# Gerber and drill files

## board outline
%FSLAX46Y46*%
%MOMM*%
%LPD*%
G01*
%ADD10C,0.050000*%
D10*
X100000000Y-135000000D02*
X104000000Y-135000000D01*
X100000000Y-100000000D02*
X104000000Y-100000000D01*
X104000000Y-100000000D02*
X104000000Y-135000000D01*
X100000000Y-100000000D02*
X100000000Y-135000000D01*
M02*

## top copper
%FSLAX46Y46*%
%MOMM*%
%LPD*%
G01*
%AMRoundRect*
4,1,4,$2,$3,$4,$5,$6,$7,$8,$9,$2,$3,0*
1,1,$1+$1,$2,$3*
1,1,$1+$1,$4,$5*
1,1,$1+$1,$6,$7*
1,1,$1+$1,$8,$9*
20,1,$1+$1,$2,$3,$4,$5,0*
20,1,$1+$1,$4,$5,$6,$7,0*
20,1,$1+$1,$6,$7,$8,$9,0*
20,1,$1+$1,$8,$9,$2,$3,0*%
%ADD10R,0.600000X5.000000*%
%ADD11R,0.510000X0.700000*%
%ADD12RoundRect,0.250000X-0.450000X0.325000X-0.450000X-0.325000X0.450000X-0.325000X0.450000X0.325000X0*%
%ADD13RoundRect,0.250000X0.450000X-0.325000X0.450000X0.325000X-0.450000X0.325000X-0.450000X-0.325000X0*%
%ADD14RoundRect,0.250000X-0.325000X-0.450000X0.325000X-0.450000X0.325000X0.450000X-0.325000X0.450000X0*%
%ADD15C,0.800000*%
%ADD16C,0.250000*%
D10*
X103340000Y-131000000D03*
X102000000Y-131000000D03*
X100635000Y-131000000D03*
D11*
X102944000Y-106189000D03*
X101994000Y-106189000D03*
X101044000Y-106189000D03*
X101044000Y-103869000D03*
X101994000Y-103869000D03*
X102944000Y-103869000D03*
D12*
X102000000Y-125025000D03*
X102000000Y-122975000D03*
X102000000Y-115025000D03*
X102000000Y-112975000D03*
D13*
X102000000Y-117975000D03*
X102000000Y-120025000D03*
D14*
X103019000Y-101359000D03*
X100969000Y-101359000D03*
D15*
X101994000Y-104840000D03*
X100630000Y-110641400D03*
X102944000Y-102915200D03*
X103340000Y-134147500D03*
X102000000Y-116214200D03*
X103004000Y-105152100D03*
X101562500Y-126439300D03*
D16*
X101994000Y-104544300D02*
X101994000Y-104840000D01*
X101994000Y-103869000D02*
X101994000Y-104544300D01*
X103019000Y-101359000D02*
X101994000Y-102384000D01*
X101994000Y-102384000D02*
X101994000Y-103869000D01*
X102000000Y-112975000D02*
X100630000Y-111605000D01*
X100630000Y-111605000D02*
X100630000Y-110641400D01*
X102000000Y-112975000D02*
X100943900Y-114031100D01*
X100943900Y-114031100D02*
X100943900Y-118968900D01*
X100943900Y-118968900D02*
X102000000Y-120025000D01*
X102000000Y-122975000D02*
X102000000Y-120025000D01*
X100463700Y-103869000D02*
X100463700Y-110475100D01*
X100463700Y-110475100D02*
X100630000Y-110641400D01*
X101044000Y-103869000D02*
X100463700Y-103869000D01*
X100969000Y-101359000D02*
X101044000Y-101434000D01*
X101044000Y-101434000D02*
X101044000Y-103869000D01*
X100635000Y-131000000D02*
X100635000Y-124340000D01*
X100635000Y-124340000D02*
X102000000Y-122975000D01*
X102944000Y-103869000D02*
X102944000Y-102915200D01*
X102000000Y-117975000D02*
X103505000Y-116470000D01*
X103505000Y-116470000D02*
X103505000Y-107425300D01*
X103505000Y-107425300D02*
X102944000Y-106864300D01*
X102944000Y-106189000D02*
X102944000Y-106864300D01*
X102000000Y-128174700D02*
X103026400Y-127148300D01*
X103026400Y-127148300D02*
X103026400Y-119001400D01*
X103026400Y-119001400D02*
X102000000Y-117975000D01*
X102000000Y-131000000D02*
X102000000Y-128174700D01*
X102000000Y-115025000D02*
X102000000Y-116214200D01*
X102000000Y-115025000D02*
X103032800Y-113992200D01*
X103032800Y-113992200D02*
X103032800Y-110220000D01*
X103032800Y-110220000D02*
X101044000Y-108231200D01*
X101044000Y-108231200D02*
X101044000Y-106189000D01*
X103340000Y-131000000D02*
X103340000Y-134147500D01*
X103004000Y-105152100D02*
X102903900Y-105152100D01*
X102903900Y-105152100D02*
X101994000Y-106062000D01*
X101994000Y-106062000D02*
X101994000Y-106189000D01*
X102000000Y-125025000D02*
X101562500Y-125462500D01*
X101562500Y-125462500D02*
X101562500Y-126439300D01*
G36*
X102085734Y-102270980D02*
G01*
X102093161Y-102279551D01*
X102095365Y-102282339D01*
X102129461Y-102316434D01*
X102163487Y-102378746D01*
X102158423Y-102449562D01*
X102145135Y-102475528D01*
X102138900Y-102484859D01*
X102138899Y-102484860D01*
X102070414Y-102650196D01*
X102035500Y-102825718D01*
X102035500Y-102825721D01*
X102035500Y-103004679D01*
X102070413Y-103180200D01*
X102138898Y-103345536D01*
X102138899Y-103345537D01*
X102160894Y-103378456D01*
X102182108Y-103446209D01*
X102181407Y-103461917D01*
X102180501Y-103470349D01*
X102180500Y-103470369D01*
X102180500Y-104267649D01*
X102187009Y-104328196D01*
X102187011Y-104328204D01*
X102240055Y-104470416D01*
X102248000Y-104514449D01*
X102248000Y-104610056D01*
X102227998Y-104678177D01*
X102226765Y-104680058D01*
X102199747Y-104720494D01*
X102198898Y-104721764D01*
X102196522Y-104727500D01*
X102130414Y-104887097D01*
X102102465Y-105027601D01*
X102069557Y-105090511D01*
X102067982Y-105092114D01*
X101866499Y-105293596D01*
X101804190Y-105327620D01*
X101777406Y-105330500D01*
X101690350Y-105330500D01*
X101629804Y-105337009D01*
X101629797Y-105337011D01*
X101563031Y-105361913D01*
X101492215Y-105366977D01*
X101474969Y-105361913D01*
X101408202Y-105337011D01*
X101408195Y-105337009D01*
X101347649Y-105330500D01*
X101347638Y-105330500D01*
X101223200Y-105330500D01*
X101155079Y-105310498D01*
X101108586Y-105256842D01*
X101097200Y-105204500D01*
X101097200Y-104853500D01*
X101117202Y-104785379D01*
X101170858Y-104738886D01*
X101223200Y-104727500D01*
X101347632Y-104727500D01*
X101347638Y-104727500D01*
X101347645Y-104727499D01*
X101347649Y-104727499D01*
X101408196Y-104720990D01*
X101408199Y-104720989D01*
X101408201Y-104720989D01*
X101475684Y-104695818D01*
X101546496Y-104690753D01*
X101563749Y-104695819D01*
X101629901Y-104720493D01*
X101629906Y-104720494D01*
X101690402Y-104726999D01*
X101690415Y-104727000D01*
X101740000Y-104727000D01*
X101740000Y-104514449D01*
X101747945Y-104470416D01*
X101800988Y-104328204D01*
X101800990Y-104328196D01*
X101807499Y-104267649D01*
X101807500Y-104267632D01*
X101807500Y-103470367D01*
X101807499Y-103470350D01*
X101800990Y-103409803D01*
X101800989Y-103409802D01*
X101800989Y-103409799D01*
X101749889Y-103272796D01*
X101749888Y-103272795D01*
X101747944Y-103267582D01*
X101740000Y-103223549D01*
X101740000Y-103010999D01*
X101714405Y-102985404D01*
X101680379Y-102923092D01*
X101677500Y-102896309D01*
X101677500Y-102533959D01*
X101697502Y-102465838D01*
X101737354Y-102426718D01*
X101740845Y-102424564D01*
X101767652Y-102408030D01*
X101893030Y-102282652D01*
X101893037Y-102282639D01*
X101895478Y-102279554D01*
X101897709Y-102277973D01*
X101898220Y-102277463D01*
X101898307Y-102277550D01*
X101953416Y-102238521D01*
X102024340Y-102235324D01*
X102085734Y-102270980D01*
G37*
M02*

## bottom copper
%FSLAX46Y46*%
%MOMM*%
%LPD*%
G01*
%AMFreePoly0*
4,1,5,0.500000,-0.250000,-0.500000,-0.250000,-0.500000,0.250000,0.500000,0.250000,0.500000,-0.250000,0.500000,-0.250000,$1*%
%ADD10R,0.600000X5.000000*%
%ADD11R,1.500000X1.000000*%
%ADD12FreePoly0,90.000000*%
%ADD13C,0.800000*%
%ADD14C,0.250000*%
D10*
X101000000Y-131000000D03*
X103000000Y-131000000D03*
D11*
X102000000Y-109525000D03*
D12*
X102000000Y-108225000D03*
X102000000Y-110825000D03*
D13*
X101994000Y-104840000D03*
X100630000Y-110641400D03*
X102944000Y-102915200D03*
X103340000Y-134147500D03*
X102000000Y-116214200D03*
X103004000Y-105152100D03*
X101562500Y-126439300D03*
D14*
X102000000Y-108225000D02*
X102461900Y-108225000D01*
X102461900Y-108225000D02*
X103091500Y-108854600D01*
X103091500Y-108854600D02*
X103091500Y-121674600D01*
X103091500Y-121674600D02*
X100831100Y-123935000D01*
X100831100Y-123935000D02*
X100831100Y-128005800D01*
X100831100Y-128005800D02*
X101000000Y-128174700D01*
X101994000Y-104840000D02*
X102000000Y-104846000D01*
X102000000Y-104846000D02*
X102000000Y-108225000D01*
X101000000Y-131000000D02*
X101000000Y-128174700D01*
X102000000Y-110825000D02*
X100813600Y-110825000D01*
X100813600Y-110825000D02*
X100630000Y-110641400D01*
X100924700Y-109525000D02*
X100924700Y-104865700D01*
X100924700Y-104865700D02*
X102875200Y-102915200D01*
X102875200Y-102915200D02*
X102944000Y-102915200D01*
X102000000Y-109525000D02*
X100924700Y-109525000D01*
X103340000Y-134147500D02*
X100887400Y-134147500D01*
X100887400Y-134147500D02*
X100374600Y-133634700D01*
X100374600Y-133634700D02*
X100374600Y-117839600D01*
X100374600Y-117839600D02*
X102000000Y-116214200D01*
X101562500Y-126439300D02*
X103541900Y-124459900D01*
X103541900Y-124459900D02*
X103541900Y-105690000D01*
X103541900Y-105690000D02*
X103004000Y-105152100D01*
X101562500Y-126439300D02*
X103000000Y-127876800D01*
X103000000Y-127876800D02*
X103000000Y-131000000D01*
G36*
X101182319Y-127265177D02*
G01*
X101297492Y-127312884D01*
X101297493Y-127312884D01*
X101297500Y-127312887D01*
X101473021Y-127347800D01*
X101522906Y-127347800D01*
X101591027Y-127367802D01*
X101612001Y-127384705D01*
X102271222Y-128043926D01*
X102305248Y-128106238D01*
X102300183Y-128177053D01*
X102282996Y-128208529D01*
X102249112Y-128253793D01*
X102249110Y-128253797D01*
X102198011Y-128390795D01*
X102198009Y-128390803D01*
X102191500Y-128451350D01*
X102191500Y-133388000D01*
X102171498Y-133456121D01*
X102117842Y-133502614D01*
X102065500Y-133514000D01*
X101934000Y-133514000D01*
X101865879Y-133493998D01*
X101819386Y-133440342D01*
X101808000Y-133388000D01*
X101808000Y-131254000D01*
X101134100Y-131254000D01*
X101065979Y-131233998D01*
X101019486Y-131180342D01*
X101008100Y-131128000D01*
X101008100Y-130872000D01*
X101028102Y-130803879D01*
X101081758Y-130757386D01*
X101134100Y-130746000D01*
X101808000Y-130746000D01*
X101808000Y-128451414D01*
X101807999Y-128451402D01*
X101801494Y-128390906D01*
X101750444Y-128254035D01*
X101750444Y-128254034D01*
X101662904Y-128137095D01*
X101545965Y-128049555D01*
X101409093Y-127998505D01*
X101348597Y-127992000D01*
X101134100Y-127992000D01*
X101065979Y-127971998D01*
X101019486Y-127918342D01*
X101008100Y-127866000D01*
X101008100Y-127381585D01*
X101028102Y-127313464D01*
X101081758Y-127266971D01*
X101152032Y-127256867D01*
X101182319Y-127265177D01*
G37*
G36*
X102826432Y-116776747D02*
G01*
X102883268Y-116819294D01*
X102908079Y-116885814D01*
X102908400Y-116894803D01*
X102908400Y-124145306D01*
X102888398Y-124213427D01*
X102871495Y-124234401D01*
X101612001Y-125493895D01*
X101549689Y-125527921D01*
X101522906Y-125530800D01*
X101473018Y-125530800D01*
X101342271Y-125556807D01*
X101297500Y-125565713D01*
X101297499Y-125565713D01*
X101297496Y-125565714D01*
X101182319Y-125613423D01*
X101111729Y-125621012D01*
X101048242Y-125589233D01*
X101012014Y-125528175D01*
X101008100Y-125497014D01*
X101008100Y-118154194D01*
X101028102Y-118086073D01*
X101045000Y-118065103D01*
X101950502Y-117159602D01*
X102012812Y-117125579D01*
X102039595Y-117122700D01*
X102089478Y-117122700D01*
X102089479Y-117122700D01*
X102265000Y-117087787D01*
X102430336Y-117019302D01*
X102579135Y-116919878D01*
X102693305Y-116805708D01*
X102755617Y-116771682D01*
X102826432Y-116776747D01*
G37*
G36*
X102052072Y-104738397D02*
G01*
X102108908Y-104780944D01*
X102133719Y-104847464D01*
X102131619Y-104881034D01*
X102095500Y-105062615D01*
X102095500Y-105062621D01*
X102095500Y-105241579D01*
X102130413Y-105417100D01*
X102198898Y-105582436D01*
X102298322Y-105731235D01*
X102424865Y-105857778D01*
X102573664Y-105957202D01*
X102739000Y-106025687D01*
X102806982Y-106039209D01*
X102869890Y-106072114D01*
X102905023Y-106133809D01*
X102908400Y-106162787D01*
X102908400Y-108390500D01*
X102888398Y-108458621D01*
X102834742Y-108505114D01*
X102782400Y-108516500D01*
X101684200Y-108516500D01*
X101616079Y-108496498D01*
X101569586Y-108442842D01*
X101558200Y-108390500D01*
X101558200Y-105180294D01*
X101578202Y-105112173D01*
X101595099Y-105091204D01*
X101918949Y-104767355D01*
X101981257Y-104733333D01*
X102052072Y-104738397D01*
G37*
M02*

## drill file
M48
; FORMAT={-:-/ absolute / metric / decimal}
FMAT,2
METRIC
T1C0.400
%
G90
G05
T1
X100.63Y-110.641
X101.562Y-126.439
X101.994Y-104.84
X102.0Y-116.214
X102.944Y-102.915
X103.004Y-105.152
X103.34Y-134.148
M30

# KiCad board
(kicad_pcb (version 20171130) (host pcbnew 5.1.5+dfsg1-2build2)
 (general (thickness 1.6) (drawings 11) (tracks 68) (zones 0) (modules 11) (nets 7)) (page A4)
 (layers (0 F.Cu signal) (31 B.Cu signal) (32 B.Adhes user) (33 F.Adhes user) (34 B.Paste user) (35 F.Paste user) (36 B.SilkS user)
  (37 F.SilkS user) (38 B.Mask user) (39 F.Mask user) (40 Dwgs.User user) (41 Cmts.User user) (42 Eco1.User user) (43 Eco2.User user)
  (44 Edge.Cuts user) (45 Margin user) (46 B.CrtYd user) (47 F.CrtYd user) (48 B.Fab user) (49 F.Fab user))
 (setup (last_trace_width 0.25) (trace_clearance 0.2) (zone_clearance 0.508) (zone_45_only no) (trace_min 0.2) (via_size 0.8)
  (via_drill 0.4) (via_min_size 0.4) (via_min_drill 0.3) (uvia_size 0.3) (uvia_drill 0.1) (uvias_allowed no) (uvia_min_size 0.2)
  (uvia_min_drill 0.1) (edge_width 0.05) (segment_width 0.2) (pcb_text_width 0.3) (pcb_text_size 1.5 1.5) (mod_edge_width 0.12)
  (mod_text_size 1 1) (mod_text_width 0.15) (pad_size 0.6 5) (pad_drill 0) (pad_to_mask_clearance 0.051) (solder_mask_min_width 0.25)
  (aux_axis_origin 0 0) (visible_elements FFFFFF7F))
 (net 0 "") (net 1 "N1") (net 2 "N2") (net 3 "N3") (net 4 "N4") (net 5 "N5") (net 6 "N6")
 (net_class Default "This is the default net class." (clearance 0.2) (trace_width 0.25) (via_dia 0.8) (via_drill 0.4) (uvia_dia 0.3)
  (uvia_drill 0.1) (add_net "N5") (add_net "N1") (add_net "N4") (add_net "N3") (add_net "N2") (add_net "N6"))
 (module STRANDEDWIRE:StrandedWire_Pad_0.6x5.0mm (layer B.Cu) (at 101 131)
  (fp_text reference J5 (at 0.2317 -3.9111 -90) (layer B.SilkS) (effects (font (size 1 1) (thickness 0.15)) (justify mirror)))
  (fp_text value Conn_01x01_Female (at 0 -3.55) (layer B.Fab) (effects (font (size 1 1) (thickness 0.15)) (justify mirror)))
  (pad 1 smd rect (at 0 0) (size 0.6 5) (layers B.Cu B.Mask) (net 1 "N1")))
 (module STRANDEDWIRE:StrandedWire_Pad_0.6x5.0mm (layer B.Cu) (at 103 131)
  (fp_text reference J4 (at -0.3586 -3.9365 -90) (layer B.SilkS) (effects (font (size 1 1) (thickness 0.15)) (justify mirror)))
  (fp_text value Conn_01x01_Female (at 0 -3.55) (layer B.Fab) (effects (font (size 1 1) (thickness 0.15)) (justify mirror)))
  (pad 1 smd rect (at 0 0) (size 0.6 5) (layers B.Cu B.Mask) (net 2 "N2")))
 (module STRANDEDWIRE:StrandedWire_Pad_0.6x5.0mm (layer F.Cu) (at 103.34 131)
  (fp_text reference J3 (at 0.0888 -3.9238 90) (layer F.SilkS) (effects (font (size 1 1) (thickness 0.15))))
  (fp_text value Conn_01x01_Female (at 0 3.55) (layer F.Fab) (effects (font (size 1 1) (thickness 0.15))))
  (pad 1 smd rect (at 0 0) (size 0.6 5) (layers F.Cu F.Mask) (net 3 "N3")))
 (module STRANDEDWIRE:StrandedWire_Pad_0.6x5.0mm (layer F.Cu) (at 102 131)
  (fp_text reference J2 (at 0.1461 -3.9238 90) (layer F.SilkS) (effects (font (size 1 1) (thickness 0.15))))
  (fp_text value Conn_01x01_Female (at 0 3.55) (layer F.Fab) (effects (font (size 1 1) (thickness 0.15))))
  (pad 1 smd rect (at 0 0) (size 0.6 5) (layers F.Cu F.Mask) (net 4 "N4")))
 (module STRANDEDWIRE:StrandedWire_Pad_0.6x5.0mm (layer F.Cu) (at 100.635 131)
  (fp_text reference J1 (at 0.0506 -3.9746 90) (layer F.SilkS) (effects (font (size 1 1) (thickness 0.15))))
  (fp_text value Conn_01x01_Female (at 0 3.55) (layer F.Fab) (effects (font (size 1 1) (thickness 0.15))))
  (pad 1 smd rect (at 0 0) (size 0.6 5) (layers F.Cu F.Mask) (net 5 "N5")))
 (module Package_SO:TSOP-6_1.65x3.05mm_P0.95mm (layer F.Cu) (at 101.994 105.029 270)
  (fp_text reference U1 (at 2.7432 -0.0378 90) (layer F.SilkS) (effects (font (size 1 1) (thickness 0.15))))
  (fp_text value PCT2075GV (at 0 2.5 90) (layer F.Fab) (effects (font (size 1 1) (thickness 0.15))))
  (pad 6 smd rect (at 1.16 -0.95 270) (size 0.7 0.51) (layers F.Cu F.Paste F.Mask) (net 4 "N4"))
  (pad 5 smd rect (at 1.16 0 270) (size 0.7 0.51) (layers F.Cu F.Paste F.Mask) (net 2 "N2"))
  (pad 4 smd rect (at 1.16 0.95 270) (size 0.7 0.51) (layers F.Cu F.Paste F.Mask) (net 3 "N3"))
  (pad 3 smd rect (at -1.16 0.95 270) (size 0.7 0.51) (layers F.Cu F.Paste F.Mask) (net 5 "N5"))
  (pad 2 smd rect (at -1.16 0 270) (size 0.7 0.51) (layers F.Cu F.Paste F.Mask) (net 1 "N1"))
  (pad 1 smd rect (at -1.16 -0.95 270) (size 0.7 0.51) (layers F.Cu F.Paste F.Mask) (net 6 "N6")))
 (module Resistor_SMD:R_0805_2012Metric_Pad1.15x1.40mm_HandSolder (layer F.Cu) (at 102 124 270)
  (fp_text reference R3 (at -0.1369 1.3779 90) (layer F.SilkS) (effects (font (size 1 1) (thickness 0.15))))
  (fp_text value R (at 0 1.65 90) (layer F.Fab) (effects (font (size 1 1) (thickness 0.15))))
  (pad 2 smd roundrect (at 1.025 0 270) (size 1.15 1.4) (layers F.Cu F.Paste F.Mask) (roundrect_rratio 0.217391) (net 2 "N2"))
  (pad 1 smd roundrect (at -1.025 0 270) (size 1.15 1.4) (layers F.Cu F.Paste F.Mask) (roundrect_rratio 0.217391) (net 5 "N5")))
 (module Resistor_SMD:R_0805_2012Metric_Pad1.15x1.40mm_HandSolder (layer F.Cu) (at 102 114 270)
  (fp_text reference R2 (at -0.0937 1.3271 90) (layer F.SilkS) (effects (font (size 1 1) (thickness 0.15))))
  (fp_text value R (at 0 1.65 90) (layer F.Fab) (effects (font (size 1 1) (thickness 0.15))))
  (pad 2 smd roundrect (at 1.025 0 270) (size 1.15 1.4) (layers F.Cu F.Paste F.Mask) (roundrect_rratio 0.217391) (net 3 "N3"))
  (pad 1 smd roundrect (at -1.025 0 270) (size 1.15 1.4) (layers F.Cu F.Paste F.Mask) (roundrect_rratio 0.217391) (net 5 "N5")))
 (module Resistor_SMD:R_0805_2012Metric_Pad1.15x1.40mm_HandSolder (layer F.Cu) (at 102 119 90)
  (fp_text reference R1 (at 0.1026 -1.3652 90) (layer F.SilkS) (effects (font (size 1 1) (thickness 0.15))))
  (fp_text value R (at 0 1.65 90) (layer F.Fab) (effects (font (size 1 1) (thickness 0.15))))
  (pad 2 smd roundrect (at 1.025 0 90) (size 1.15 1.4) (layers F.Cu F.Paste F.Mask) (roundrect_rratio 0.217391) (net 4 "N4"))
  (pad 1 smd roundrect (at -1.025 0 90) (size 1.15 1.4) (layers F.Cu F.Paste F.Mask) (roundrect_rratio 0.217391) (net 5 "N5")))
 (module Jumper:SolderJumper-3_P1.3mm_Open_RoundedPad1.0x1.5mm (layer B.Cu) (at 102 109.525 90)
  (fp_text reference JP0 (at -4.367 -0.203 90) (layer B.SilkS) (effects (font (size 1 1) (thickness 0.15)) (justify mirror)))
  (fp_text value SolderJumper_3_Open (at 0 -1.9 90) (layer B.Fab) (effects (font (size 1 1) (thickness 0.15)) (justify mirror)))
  (pad 2 smd rect (at 0 0 90) (size 1 1.5) (layers B.Cu B.Mask) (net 6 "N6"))
  (pad 3 smd custom (at 1.3 0 90) (size 1 0.5) (layers B.Cu B.Mask) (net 1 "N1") (zone_connect 2)
   (options (clearance outline) (anchor rect)) (primitives))
  (pad 1 smd custom (at -1.3 0 90) (size 1 0.5) (layers B.Cu B.Mask) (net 5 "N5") (zone_connect 2)
   (options (clearance outline) (anchor rect)) (primitives)))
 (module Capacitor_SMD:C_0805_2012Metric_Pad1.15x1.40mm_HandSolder (layer F.Cu) (at 101.994 101.359)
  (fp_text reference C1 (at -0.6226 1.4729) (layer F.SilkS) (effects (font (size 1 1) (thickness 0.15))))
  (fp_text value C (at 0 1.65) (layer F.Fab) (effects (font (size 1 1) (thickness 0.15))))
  (pad 2 smd roundrect (at 1.025 0) (size 1.15 1.4) (layers F.Cu F.Paste F.Mask) (roundrect_rratio 0.217391) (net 1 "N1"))
  (pad 1 smd roundrect (at -1.025 0) (size 1.15 1.4) (layers F.Cu F.Paste F.Mask) (roundrect_rratio 0.217391) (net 5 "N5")))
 (gr_line (start 100 135) (end 104 135) (layer Edge.Cuts) (width 0.05))
 (gr_line (start 100 100) (end 104 100) (layer Edge.Cuts) (width 0.05))
 (gr_line (start 104 100) (end 104 135) (layer Edge.Cuts) (width 0.05))
 (gr_line (start 100 100) (end 100 135) (layer Edge.Cuts) (width 0.05))
 (segment (start 102 108.225) (end 102.4619 108.225) (width 0.25) (layer B.Cu) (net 1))
 (segment (start 102.4619 108.225) (end 103.0915 108.8546) (width 0.25) (layer B.Cu) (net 1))
 (segment (start 103.0915 108.8546) (end 103.0915 121.6746) (width 0.25) (layer B.Cu) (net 1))
 (segment (start 103.0915 121.6746) (end 100.8311 123.935) (width 0.25) (layer B.Cu) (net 1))
 (segment (start 100.8311 123.935) (end 100.8311 128.0058) (width 0.25) (layer B.Cu) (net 1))
 (segment (start 100.8311 128.0058) (end 101 128.1747) (width 0.25) (layer B.Cu) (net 1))
 (segment (start 101.994 104.84) (end 102 104.846) (width 0.25) (layer B.Cu) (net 1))
 (segment (start 102 104.846) (end 102 108.225) (width 0.25) (layer B.Cu) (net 1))
 (segment (start 101 131) (end 101 128.1747) (width 0.25) (layer B.Cu) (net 1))
 (segment (start 101.994 104.5443) (end 101.994 104.84) (width 0.25) (layer F.Cu) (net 1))
 (segment (start 101.994 103.869) (end 101.994 104.5443) (width 0.25) (layer F.Cu) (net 1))
 (segment (start 103.019 101.359) (end 101.994 102.384) (width 0.25) (layer F.Cu) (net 1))
 (segment (start 101.994 102.384) (end 101.994 103.869) (width 0.25) (layer F.Cu) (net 1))
 (via (at 101.994 104.84) (size 0.8) (layers F.Cu B.Cu) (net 1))
 (segment (start 102 112.975) (end 100.63 111.605) (width 0.25) (layer F.Cu) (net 5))
 (segment (start 100.63 111.605) (end 100.63 110.6414) (width 0.25) (layer F.Cu) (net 5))
 (segment (start 102 112.975) (end 100.9439 114.0311) (width 0.25) (layer F.Cu) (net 5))
 (segment (start 100.9439 114.0311) (end 100.9439 118.9689) (width 0.25) (layer F.Cu) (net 5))
 (segment (start 100.9439 118.9689) (end 102 120.025) (width 0.25) (layer F.Cu) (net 5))
 (segment (start 102 122.975) (end 102 120.025) (width 0.25) (layer F.Cu) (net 5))
 (segment (start 100.4637 103.869) (end 100.4637 110.4751) (width 0.25) (layer F.Cu) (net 5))
 (segment (start 100.4637 110.4751) (end 100.63 110.6414) (width 0.25) (layer F.Cu) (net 5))
 (segment (start 101.044 103.869) (end 100.4637 103.869) (width 0.25) (layer F.Cu) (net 5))
 (segment (start 100.969 101.359) (end 101.044 101.434) (width 0.25) (layer F.Cu) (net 5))
 (segment (start 101.044 101.434) (end 101.044 103.869) (width 0.25) (layer F.Cu) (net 5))
 (segment (start 102 110.825) (end 100.8136 110.825) (width 0.25) (layer B.Cu) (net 5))
 (segment (start 100.8136 110.825) (end 100.63 110.6414) (width 0.25) (layer B.Cu) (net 5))
 (segment (start 100.635 131) (end 100.635 124.34) (width 0.25) (layer F.Cu) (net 5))
 (segment (start 100.635 124.34) (end 102 122.975) (width 0.25) (layer F.Cu) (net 5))
 (via (at 100.63 110.6414) (size 0.8) (layers F.Cu B.Cu) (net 5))
 (segment (start 102.944 103.869) (end 102.944 102.9152) (width 0.25) (layer F.Cu) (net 6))
 (segment (start 100.9247 109.525) (end 100.9247 104.8657) (width 0.25) (layer B.Cu) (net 6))
 (segment (start 100.9247 104.8657) (end 102.8752 102.9152) (width 0.25) (layer B.Cu) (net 6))
 (segment (start 102.8752 102.9152) (end 102.944 102.9152) (width 0.25) (layer B.Cu) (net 6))
 (segment (start 102 109.525) (end 100.9247 109.525) (width 0.25) (layer B.Cu) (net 6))
 (via (at 102.944 102.9152) (size 0.8) (layers F.Cu B.Cu) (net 6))
 (segment (start 102 117.975) (end 103.505 116.47) (width 0.25) (layer F.Cu) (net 4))
 (segment (start 103.505 116.47) (end 103.505 107.4253) (width 0.25) (layer F.Cu) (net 4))
 (segment (start 103.505 107.4253) (end 102.944 106.8643) (width 0.25) (layer F.Cu) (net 4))
 (segment (start 102.944 106.189) (end 102.944 106.8643) (width 0.25) (layer F.Cu) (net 4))
 (segment (start 102 128.1747) (end 103.0264 127.1483) (width 0.25) (layer F.Cu) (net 4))
 (segment (start 103.0264 127.1483) (end 103.0264 119.0014) (width 0.25) (layer F.Cu) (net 4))
 (segment (start 103.0264 119.0014) (end 102 117.975) (width 0.25) (layer F.Cu) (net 4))
 (segment (start 102 131) (end 102 128.1747) (width 0.25) (layer F.Cu) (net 4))
 (segment (start 102 115.025) (end 102 116.2142) (width 0.25) (layer F.Cu) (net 3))
 (segment (start 103.34 134.1475) (end 100.8874 134.1475) (width 0.25) (layer B.Cu) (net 3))
 (segment (start 100.8874 134.1475) (end 100.3746 133.6347) (width 0.25) (layer B.Cu) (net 3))
 (segment (start 100.3746 133.6347) (end 100.3746 117.8396) (width 0.25) (layer B.Cu) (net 3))
 (segment (start 100.3746 117.8396) (end 102 116.2142) (width 0.25) (layer B.Cu) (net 3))
 (segment (start 102 115.025) (end 103.0328 113.9922) (width 0.25) (layer F.Cu) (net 3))
 (segment (start 103.0328 113.9922) (end 103.0328 110.22) (width 0.25) (layer F.Cu) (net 3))
 (segment (start 103.0328 110.22) (end 101.044 108.2312) (width 0.25) (layer F.Cu) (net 3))
 (segment (start 101.044 108.2312) (end 101.044 106.189) (width 0.25) (layer F.Cu) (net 3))
 (segment (start 103.34 131) (end 103.34 134.1475) (width 0.25) (layer F.Cu) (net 3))
 (via (at 103.34 134.1475) (size 0.8) (layers F.Cu B.Cu) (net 3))
 (via (at 102 116.2142) (size 0.8) (layers F.Cu B.Cu) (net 3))
 (segment (start 101.5625 126.4393) (end 103.5419 124.4599) (width 0.25) (layer B.Cu) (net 2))
 (segment (start 103.5419 124.4599) (end 103.5419 105.69) (width 0.25) (layer B.Cu) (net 2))
 (segment (start 103.5419 105.69) (end 103.004 105.1521) (width 0.25) (layer B.Cu) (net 2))
 (segment (start 103.004 105.1521) (end 102.9039 105.1521) (width 0.25) (layer F.Cu) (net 2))
 (segment (start 102.9039 105.1521) (end 101.994 106.062) (width 0.25) (layer F.Cu) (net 2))
 (segment (start 101.994 106.062) (end 101.994 106.189) (width 0.25) (layer F.Cu) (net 2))
 (segment (start 101.5625 126.4393) (end 103 127.8768) (width 0.25) (layer B.Cu) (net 2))
 (segment (start 103 127.8768) (end 103 131) (width 0.25) (layer B.Cu) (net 2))
 (segment (start 102 125.025) (end 101.5625 125.4625) (width 0.25) (layer F.Cu) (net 2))
 (segment (start 101.5625 125.4625) (end 101.5625 126.4393) (width 0.25) (layer F.Cu) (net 2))
 (via (at 103.004 105.1521) (size 0.8) (layers F.Cu B.Cu) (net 2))
 (via (at 101.5625 126.4393) (size 0.8) (layers F.Cu B.Cu) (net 2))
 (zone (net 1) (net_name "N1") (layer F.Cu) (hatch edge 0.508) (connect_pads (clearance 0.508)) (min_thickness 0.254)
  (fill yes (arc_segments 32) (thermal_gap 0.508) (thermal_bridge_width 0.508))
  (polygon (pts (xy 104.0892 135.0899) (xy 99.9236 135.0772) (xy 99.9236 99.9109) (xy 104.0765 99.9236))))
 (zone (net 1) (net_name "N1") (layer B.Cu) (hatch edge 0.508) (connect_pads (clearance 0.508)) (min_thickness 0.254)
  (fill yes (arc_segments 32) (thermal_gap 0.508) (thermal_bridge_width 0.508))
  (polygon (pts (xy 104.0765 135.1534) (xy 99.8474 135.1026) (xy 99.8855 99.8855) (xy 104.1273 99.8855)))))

